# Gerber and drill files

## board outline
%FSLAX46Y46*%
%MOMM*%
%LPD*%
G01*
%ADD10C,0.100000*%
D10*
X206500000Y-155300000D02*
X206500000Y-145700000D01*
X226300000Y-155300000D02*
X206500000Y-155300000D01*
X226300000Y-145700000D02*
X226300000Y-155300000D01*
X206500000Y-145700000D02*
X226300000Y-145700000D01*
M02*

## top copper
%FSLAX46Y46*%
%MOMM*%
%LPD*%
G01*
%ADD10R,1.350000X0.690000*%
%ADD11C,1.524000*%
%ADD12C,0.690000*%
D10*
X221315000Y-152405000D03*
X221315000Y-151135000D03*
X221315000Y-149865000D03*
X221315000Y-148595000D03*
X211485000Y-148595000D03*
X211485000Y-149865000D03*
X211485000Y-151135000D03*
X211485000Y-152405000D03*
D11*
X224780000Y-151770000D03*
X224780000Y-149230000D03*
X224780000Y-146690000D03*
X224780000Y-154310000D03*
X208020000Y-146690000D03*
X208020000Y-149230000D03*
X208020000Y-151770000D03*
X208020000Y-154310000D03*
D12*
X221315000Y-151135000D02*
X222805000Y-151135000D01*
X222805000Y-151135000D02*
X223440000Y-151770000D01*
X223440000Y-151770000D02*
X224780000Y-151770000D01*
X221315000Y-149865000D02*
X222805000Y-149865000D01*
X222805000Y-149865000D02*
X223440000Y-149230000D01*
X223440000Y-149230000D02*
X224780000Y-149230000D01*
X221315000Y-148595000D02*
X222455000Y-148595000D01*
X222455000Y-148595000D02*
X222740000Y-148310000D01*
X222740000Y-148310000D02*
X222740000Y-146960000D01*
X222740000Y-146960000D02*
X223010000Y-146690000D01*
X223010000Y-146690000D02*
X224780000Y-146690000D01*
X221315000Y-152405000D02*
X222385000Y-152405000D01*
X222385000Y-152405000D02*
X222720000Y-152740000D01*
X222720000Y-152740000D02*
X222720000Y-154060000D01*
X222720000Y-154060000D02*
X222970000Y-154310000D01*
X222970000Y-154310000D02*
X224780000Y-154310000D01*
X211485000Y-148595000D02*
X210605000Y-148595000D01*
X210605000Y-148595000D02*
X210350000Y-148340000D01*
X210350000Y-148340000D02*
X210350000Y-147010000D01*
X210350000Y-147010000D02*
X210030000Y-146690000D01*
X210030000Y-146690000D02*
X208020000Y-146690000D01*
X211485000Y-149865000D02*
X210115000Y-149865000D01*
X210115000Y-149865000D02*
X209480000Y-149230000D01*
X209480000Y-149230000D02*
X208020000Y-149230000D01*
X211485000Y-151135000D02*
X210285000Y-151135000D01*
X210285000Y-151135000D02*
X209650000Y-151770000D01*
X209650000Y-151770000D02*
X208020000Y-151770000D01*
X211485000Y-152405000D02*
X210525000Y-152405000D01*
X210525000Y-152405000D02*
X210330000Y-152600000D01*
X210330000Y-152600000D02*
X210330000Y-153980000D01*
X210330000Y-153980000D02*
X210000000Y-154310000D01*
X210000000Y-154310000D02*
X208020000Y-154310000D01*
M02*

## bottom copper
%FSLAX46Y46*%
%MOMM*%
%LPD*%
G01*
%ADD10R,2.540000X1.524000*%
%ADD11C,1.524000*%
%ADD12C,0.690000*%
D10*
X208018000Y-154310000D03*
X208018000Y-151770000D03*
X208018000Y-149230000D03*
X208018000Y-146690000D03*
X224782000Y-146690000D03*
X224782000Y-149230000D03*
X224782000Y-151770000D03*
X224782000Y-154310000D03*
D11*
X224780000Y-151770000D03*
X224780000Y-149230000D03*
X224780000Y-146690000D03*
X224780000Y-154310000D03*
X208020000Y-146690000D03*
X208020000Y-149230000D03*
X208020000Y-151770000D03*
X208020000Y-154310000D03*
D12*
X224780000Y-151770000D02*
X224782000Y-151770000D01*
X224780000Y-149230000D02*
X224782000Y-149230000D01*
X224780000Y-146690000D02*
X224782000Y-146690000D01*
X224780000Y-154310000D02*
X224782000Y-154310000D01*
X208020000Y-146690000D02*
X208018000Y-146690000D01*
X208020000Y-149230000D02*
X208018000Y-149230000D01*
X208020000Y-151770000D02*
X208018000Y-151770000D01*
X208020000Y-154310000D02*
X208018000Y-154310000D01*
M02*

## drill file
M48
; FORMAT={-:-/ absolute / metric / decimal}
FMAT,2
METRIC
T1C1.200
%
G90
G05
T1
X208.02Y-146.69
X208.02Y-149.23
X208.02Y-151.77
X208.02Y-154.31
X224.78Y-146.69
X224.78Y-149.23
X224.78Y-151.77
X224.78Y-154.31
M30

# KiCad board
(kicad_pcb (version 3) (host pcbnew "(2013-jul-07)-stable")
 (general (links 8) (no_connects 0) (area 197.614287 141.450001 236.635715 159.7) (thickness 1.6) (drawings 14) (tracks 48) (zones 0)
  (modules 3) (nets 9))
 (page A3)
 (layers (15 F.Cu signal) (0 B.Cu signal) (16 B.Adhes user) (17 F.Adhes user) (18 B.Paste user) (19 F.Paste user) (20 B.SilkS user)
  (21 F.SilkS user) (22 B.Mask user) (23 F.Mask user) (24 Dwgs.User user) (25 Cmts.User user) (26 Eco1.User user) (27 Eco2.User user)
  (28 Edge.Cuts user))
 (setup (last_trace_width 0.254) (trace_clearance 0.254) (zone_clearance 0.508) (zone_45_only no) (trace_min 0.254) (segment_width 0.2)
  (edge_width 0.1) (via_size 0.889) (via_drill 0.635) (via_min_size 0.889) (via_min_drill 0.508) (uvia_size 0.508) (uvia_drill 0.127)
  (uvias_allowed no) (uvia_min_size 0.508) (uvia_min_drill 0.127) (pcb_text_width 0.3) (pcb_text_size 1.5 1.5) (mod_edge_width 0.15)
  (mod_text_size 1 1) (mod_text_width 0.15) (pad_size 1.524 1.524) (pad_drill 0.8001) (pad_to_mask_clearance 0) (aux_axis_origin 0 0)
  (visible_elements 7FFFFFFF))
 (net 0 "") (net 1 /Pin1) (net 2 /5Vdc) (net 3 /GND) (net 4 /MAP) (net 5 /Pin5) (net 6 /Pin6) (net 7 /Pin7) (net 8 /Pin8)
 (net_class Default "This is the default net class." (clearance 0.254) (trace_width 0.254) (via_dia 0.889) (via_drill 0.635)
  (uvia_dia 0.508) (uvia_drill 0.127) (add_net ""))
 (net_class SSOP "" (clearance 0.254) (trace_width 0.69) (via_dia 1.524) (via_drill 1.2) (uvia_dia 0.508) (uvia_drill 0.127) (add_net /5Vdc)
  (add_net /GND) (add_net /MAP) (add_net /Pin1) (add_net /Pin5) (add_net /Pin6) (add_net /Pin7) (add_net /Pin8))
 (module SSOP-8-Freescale (layer F.Cu) (at 216.4 150.5)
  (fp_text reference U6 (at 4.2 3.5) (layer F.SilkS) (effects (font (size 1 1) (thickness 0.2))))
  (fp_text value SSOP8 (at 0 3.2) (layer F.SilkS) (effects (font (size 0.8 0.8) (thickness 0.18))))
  (pad 1 smd rect (at 4.915 1.905) (size 1.35 0.69) (layers F.Cu F.Paste F.Mask) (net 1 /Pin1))
  (pad 2 smd rect (at 4.915 0.635) (size 1.35 0.69) (layers F.Cu F.Paste F.Mask) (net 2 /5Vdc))
  (pad 3 smd rect (at 4.915 -0.635) (size 1.35 0.69) (layers F.Cu F.Paste F.Mask) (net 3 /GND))
  (pad 4 smd rect (at 4.915 -1.905) (size 1.35 0.69) (layers F.Cu F.Paste F.Mask) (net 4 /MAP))
  (pad 5 smd rect (at -4.915 -1.905) (size 1.35 0.69) (layers F.Cu F.Paste F.Mask) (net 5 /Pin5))
  (pad 6 smd rect (at -4.915 -0.635) (size 1.35 0.69) (layers F.Cu F.Paste F.Mask) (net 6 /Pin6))
  (pad 7 smd rect (at -4.915 0.635) (size 1.35 0.69) (layers F.Cu F.Paste F.Mask) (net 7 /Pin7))
  (pad 8 smd rect (at -4.915 1.905) (size 1.35 0.69) (layers F.Cu F.Paste F.Mask) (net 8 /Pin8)))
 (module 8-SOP (layer B.Cu) (at 216.4 150.5 180)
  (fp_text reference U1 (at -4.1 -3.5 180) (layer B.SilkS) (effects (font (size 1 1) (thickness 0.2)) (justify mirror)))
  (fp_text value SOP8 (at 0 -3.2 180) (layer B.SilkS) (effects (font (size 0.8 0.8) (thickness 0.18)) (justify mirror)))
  (pad 1 smd rect (at 8.382 -3.81 180) (size 2.54 1.524) (layers B.Cu B.Paste B.Mask) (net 8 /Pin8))
  (pad 2 smd rect (at 8.382 -1.27 180) (size 2.54 1.524) (layers B.Cu B.Paste B.Mask) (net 7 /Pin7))
  (pad 3 smd rect (at 8.382 1.27 180) (size 2.54 1.524) (layers B.Cu B.Paste B.Mask) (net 6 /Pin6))
  (pad 4 smd rect (at 8.382 3.81 180) (size 2.54 1.524) (layers B.Cu B.Paste B.Mask) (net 5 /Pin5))
  (pad 5 smd rect (at -8.382 3.81 180) (size 2.54 1.524) (layers B.Cu B.Paste B.Mask) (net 4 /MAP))
  (pad 6 smd rect (at -8.382 1.27 180) (size 2.54 1.524) (layers B.Cu B.Paste B.Mask) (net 3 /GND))
  (pad 7 smd rect (at -8.382 -1.27 180) (size 2.54 1.524) (layers B.Cu B.Paste B.Mask) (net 2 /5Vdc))
  (pad 8 smd rect (at -8.382 -3.81 180) (size 2.54 1.524) (layers B.Cu B.Paste B.Mask) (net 1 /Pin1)))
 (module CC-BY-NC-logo (layer F.Cu) (at 219.4 146.7)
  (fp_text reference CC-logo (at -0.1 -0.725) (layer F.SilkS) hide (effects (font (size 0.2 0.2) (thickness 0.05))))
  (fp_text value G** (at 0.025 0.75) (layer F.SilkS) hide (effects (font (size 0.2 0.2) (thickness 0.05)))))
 (gr_line (start 206.5 155.3) (end 206.5 145.7) (angle 90) (layer Edge.Cuts) (width 0.1))
 (gr_line (start 226.3 155.3) (end 206.5 155.3) (angle 90) (layer Edge.Cuts) (width 0.1))
 (gr_line (start 226.3 145.7) (end 226.3 155.3) (angle 90) (layer Edge.Cuts) (width 0.1))
 (gr_line (start 206.5 145.7) (end 226.3 145.7) (angle 90) (layer Edge.Cuts) (width 0.1))
 (segment (start 221.315 151.135) (end 222.805 151.135) (width 0.69) (layer F.Cu) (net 2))
 (segment (start 222.805 151.135) (end 223.44 151.77) (width 0.69) (layer F.Cu) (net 2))
 (segment (start 223.44 151.77) (end 224.78 151.77) (width 0.69) (layer F.Cu) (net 2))
 (via (at 224.78 151.77) (size 1.524) (layers F.Cu B.Cu) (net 2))
 (segment (start 224.78 151.77) (end 224.782 151.77) (width 0.69) (layer B.Cu) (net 2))
 (segment (start 221.315 149.865) (end 222.805 149.865) (width 0.69) (layer F.Cu) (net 3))
 (segment (start 222.805 149.865) (end 223.44 149.23) (width 0.69) (layer F.Cu) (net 3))
 (segment (start 223.44 149.23) (end 224.78 149.23) (width 0.69) (layer F.Cu) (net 3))
 (via (at 224.78 149.23) (size 1.524) (layers F.Cu B.Cu) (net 3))
 (segment (start 224.78 149.23) (end 224.782 149.23) (width 0.69) (layer B.Cu) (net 3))
 (segment (start 221.315 148.595) (end 222.455 148.595) (width 0.69) (layer F.Cu) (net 4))
 (segment (start 222.455 148.595) (end 222.74 148.31) (width 0.69) (layer F.Cu) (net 4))
 (segment (start 222.74 148.31) (end 222.74 146.96) (width 0.69) (layer F.Cu) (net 4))
 (segment (start 222.74 146.96) (end 223.01 146.69) (width 0.69) (layer F.Cu) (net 4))
 (segment (start 223.01 146.69) (end 224.78 146.69) (width 0.69) (layer F.Cu) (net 4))
 (via (at 224.78 146.69) (size 1.524) (layers F.Cu B.Cu) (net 4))
 (segment (start 224.78 146.69) (end 224.782 146.69) (width 0.69) (layer B.Cu) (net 4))
 (segment (start 221.315 152.405) (end 222.385 152.405) (width 0.69) (layer F.Cu) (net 1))
 (segment (start 222.385 152.405) (end 222.72 152.74) (width 0.69) (layer F.Cu) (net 1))
 (segment (start 222.72 152.74) (end 222.72 154.06) (width 0.69) (layer F.Cu) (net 1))
 (segment (start 222.72 154.06) (end 222.97 154.31) (width 0.69) (layer F.Cu) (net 1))
 (segment (start 222.97 154.31) (end 224.78 154.31) (width 0.69) (layer F.Cu) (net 1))
 (via (at 224.78 154.31) (size 1.524) (layers F.Cu B.Cu) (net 1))
 (segment (start 224.78 154.31) (end 224.782 154.31) (width 0.69) (layer B.Cu) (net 1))
 (segment (start 211.485 148.595) (end 210.605 148.595) (width 0.69) (layer F.Cu) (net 5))
 (segment (start 210.605 148.595) (end 210.35 148.34) (width 0.69) (layer F.Cu) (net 5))
 (segment (start 210.35 148.34) (end 210.35 147.01) (width 0.69) (layer F.Cu) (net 5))
 (segment (start 210.35 147.01) (end 210.03 146.69) (width 0.69) (layer F.Cu) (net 5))
 (segment (start 210.03 146.69) (end 208.02 146.69) (width 0.69) (layer F.Cu) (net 5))
 (via (at 208.02 146.69) (size 1.524) (layers F.Cu B.Cu) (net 5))
 (segment (start 208.02 146.69) (end 208.018 146.69) (width 0.69) (layer B.Cu) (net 5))
 (segment (start 211.485 149.865) (end 210.115 149.865) (width 0.69) (layer F.Cu) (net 6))
 (segment (start 210.115 149.865) (end 209.48 149.23) (width 0.69) (layer F.Cu) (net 6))
 (segment (start 209.48 149.23) (end 208.02 149.23) (width 0.69) (layer F.Cu) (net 6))
 (via (at 208.02 149.23) (size 1.524) (layers F.Cu B.Cu) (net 6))
 (segment (start 208.02 149.23) (end 208.018 149.23) (width 0.69) (layer B.Cu) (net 6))
 (segment (start 211.485 151.135) (end 210.285 151.135) (width 0.69) (layer F.Cu) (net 7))
 (segment (start 210.285 151.135) (end 209.65 151.77) (width 0.69) (layer F.Cu) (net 7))
 (segment (start 209.65 151.77) (end 208.02 151.77) (width 0.69) (layer F.Cu) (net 7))
 (via (at 208.02 151.77) (size 1.524) (layers F.Cu B.Cu) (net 7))
 (segment (start 208.02 151.77) (end 208.018 151.77) (width 0.69) (layer B.Cu) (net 7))
 (segment (start 211.485 152.405) (end 210.525 152.405) (width 0.69) (layer F.Cu) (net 8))
 (segment (start 210.525 152.405) (end 210.33 152.6) (width 0.69) (layer F.Cu) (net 8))
 (segment (start 210.33 152.6) (end 210.33 153.98) (width 0.69) (layer F.Cu) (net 8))
 (segment (start 210.33 153.98) (end 210 154.31) (width 0.69) (layer F.Cu) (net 8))
 (segment (start 210 154.31) (end 208.02 154.31) (width 0.69) (layer F.Cu) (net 8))
 (via (at 208.02 154.31) (size 1.524) (layers F.Cu B.Cu) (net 8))
 (segment (start 208.02 154.31) (end 208.018 154.31) (width 0.69) (layer B.Cu) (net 8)))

